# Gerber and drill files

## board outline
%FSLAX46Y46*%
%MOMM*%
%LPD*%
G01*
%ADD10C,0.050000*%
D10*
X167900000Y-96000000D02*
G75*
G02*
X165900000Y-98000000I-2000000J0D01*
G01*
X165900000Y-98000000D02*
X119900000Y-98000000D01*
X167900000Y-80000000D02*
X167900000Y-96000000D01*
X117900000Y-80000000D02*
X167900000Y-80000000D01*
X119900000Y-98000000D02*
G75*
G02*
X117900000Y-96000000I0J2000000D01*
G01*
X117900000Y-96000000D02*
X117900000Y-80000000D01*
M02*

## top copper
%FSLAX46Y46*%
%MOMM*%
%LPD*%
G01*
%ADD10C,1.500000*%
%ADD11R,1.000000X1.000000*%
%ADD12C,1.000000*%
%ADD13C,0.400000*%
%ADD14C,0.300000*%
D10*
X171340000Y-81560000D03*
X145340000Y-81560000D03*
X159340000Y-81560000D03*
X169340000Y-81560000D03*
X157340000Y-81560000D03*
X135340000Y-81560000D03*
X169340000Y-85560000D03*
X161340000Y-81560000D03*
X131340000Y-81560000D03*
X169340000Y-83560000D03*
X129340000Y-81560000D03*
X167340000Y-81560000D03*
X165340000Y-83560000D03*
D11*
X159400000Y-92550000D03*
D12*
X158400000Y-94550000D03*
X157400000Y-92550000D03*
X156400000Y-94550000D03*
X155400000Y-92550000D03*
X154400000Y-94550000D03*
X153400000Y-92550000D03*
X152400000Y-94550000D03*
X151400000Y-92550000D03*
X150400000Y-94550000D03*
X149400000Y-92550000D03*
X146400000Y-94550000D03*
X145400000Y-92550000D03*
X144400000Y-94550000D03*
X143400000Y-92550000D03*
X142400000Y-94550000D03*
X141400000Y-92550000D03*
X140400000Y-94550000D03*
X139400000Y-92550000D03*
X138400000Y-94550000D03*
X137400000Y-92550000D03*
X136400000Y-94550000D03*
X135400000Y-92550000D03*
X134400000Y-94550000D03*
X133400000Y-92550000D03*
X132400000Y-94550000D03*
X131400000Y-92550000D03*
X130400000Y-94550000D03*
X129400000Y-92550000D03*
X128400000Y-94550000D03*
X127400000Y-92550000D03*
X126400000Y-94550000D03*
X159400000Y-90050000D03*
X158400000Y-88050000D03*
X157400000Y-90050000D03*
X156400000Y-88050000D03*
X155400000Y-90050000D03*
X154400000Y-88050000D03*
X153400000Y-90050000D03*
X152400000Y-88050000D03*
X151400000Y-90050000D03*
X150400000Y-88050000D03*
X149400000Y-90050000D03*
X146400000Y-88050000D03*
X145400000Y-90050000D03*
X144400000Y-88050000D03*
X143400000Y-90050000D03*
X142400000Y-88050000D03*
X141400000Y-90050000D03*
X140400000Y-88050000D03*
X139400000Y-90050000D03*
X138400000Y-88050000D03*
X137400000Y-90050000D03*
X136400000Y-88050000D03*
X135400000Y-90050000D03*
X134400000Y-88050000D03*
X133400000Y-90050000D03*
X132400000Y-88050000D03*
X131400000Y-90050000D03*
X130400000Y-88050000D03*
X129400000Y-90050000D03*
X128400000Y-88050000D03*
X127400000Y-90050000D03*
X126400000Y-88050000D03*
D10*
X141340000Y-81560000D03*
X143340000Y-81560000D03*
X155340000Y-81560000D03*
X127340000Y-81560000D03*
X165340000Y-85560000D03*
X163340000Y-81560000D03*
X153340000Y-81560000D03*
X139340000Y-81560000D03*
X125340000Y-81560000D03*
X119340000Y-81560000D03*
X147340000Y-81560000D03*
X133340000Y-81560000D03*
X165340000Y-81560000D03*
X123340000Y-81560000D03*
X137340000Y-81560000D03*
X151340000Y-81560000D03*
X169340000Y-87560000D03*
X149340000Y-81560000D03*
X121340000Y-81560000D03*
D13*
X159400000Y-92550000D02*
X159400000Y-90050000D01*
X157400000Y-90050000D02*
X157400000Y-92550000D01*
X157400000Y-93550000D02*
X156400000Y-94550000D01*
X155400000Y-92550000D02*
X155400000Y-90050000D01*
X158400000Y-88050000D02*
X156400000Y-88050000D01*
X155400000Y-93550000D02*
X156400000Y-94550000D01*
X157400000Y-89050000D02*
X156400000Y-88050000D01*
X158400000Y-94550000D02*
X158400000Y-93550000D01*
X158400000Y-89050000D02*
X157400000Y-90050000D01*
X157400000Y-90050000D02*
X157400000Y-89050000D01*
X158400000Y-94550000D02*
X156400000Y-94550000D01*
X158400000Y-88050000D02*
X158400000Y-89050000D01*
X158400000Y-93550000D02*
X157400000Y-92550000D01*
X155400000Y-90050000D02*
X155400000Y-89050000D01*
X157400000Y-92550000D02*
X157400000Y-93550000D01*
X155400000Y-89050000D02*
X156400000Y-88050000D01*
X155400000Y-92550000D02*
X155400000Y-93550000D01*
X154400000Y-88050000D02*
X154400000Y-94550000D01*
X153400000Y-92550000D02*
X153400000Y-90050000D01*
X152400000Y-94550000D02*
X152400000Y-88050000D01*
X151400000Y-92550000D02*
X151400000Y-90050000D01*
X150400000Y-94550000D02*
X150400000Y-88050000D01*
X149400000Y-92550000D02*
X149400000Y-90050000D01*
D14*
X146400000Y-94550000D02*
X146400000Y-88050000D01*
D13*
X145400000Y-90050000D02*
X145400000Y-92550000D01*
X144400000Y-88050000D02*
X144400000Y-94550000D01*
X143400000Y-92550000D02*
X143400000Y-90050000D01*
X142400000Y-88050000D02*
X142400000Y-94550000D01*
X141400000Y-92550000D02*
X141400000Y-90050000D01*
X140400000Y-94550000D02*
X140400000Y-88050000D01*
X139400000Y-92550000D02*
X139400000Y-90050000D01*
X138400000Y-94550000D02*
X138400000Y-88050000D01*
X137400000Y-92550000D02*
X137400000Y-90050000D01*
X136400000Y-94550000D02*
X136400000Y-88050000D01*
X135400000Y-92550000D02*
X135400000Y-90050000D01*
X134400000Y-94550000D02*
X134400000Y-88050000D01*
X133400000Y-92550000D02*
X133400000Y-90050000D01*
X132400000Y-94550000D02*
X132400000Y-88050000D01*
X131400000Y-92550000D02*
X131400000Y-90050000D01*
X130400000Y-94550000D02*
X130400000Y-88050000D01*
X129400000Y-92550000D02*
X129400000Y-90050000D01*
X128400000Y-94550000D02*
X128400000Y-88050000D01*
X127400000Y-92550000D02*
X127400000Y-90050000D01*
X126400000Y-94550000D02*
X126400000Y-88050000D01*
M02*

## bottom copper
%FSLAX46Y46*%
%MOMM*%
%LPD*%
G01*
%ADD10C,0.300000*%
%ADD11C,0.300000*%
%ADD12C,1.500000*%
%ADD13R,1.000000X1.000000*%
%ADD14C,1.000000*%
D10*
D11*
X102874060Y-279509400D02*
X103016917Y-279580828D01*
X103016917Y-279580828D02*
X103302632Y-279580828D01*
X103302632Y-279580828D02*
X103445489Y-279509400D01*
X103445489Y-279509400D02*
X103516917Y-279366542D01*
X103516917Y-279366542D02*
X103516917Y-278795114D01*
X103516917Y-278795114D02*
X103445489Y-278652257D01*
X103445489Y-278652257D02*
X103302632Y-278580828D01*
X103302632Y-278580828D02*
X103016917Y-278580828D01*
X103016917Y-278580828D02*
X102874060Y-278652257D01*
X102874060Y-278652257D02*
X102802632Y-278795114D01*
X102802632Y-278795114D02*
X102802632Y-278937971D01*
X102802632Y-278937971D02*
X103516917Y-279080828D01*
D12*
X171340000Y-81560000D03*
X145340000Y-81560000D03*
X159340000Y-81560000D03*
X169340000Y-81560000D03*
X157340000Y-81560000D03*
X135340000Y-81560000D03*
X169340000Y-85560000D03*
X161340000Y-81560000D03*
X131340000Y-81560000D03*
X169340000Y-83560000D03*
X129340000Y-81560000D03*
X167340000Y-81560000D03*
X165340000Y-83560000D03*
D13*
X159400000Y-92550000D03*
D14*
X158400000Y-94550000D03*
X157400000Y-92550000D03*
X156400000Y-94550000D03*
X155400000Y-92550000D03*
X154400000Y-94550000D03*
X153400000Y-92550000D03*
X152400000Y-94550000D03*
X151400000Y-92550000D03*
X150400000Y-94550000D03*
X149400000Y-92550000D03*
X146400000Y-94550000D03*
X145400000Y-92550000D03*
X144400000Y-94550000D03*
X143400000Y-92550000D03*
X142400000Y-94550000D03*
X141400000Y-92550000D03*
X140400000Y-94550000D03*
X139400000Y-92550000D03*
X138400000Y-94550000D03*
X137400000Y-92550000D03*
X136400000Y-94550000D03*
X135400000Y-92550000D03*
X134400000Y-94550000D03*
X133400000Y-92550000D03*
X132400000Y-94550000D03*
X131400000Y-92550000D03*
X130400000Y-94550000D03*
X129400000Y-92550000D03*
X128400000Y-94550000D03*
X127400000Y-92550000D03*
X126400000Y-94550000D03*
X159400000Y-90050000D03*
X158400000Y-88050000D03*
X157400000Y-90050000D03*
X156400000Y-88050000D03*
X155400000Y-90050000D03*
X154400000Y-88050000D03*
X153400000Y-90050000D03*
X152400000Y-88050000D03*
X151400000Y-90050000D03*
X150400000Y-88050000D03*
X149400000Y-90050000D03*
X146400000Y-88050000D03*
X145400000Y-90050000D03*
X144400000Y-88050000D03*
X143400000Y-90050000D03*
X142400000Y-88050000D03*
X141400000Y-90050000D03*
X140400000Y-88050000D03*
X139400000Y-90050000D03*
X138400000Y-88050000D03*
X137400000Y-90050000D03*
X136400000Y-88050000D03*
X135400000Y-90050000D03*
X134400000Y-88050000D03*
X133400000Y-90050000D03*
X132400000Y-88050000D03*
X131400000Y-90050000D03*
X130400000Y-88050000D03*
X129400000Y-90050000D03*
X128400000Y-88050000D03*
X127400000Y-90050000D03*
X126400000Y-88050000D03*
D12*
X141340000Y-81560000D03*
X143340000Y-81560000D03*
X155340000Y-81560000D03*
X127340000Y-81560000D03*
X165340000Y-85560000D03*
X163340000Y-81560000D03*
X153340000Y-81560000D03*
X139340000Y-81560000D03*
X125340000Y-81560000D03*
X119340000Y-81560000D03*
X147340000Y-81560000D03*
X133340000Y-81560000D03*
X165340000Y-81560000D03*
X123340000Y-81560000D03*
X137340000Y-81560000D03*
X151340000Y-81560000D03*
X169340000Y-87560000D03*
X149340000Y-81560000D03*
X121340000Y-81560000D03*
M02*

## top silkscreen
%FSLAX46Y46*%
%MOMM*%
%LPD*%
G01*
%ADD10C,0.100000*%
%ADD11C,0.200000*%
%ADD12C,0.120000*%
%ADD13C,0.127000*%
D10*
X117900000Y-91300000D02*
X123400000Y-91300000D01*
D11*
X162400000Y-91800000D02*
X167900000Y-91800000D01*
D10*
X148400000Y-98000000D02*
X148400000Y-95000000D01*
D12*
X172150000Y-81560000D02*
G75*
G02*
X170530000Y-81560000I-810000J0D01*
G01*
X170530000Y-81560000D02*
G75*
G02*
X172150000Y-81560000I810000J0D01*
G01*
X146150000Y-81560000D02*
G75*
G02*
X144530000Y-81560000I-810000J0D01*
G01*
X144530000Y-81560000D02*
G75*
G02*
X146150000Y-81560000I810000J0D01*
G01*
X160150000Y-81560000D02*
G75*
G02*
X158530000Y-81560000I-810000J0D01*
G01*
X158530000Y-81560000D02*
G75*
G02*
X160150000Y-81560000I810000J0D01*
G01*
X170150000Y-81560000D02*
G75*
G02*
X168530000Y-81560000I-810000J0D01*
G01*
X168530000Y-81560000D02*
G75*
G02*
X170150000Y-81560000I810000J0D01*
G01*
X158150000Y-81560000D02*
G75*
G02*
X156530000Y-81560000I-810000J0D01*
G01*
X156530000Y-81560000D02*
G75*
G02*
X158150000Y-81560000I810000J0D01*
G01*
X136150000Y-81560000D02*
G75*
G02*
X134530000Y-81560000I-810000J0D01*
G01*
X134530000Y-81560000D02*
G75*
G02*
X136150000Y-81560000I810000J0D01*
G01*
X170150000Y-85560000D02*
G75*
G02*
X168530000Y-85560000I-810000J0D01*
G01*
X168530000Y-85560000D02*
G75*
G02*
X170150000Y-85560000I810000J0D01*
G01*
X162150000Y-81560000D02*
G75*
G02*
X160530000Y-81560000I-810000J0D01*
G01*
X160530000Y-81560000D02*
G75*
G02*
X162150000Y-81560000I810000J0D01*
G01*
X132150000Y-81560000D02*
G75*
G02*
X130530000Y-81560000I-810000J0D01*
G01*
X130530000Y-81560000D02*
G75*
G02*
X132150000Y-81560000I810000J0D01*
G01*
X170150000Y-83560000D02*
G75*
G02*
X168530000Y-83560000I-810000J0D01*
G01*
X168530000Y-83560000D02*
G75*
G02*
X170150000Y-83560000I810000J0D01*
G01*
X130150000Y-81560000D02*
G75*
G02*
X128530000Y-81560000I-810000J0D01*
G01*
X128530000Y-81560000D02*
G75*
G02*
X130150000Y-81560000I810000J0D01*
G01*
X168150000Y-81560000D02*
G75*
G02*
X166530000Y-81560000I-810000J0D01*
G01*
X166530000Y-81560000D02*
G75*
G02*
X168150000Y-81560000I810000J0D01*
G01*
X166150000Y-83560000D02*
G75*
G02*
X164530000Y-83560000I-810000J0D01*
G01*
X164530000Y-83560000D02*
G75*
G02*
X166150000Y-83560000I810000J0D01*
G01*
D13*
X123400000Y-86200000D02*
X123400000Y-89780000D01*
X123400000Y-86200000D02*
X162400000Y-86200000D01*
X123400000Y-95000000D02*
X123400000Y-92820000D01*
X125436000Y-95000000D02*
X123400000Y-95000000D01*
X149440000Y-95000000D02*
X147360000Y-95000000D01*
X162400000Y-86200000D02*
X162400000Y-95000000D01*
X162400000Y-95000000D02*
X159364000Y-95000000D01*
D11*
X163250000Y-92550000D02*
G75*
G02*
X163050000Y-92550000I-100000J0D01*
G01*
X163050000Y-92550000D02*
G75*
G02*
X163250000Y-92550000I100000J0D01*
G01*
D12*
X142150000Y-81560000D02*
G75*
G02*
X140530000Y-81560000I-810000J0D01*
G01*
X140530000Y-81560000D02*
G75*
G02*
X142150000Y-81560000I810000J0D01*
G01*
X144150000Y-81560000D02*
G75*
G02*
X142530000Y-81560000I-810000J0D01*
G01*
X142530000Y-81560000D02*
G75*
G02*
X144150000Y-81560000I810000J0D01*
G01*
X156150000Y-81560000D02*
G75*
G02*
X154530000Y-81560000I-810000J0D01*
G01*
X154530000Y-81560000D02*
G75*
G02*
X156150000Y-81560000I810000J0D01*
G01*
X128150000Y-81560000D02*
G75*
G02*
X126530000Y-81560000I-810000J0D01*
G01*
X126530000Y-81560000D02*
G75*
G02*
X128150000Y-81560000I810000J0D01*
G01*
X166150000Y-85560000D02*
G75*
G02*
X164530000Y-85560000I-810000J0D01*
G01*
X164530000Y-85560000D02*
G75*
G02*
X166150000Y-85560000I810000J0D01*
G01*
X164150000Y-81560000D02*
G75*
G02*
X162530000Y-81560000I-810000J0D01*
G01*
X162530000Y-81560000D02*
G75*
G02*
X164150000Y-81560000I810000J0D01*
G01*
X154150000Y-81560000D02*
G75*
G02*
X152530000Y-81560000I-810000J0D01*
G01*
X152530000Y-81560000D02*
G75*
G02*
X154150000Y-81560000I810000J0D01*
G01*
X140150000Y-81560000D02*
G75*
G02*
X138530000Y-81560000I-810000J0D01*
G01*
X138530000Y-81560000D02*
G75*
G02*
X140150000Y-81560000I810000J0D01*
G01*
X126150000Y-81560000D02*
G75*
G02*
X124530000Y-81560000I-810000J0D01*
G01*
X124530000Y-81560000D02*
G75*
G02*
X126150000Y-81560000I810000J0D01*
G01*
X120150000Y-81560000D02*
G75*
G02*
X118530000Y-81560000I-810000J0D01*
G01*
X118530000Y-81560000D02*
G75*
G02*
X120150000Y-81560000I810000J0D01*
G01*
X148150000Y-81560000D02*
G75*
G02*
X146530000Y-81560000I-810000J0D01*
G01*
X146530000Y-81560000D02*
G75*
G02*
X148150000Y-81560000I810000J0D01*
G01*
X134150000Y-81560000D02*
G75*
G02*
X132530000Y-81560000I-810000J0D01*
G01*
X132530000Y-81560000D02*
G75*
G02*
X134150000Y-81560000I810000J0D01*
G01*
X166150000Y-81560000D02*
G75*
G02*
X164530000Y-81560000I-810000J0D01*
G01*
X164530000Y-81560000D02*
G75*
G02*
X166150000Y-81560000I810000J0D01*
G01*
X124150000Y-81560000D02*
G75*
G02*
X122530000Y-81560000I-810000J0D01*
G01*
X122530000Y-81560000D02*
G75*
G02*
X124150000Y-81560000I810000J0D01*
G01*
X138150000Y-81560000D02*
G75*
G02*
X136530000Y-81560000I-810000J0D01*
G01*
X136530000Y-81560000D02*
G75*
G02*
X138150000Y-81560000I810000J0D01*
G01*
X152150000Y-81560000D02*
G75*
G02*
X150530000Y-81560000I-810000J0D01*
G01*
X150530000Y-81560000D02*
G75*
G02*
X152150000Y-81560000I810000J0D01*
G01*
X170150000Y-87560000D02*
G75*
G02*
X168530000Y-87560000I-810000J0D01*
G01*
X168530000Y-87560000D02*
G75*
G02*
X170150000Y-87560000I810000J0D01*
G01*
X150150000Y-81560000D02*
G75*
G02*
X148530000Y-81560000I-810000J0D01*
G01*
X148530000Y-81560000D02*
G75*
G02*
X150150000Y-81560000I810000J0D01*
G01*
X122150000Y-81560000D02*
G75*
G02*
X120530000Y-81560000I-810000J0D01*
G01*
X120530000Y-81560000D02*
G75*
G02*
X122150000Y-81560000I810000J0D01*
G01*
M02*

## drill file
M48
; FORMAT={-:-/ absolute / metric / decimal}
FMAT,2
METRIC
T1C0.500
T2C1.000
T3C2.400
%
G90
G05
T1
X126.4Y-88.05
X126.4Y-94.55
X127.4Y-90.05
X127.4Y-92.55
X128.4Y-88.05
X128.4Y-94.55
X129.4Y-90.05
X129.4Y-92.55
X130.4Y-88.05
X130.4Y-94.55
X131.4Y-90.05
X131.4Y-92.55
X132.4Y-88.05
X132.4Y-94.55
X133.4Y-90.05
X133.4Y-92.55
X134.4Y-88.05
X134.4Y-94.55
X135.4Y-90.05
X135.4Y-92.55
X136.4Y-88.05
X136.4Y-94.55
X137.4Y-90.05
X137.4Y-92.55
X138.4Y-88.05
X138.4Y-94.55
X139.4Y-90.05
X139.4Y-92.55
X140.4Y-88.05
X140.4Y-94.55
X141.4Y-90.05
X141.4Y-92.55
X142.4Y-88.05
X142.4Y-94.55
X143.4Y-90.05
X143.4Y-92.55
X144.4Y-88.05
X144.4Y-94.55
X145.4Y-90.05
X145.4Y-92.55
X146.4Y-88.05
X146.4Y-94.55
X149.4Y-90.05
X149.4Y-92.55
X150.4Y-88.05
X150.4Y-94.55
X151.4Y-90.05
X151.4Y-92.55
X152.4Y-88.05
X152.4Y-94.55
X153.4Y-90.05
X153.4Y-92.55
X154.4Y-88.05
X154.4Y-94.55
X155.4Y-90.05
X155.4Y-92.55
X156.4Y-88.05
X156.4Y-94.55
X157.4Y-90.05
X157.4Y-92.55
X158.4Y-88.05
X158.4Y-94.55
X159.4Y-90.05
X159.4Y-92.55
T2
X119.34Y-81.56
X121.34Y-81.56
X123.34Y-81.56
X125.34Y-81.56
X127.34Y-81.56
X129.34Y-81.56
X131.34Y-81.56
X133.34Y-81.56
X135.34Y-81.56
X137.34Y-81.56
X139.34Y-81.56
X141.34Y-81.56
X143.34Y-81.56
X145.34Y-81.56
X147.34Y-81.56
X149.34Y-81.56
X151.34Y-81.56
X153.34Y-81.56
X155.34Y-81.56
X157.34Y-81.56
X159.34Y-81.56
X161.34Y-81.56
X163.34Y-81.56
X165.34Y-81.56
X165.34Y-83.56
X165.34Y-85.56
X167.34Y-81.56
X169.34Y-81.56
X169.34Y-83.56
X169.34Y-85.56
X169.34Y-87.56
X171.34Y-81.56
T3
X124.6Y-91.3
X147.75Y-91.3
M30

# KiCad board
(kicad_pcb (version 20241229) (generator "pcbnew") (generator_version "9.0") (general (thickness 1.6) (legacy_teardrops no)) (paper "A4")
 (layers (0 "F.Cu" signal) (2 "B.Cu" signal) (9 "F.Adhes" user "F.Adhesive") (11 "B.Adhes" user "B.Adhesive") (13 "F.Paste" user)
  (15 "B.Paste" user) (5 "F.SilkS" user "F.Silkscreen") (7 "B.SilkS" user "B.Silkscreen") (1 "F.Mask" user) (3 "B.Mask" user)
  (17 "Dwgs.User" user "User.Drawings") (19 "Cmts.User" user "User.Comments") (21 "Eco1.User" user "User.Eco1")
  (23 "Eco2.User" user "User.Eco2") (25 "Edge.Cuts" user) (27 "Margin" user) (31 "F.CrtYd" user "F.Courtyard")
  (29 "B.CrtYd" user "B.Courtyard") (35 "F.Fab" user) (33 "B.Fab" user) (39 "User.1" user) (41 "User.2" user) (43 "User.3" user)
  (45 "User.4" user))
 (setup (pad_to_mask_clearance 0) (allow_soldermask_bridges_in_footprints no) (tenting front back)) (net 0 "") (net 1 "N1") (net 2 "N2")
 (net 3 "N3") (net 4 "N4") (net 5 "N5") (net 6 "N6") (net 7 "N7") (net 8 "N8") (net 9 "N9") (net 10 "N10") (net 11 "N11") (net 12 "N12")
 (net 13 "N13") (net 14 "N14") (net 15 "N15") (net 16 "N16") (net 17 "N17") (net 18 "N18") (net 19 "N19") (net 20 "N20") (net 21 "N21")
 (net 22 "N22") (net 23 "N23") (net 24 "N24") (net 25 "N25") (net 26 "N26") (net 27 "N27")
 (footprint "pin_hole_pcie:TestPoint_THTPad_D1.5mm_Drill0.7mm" (layer "F.Cu") (at 171.34 81.56 90)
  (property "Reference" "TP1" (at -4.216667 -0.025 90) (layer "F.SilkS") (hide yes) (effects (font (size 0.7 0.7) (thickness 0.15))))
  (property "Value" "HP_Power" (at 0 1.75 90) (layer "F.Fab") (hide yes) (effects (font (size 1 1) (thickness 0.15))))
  (fp_circle (center 0 0) (end 0 0.81) (stroke (width 0.12) (type solid)) (fill no) (layer "F.SilkS"))
  (pad "1" thru_hole circle (at 0 0 90) (size 1.5 1.5) (drill 1) (layers "*.Cu" "*.Mask") (remove_unused_layers no) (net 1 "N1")))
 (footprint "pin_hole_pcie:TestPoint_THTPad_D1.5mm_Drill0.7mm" (layer "F.Cu") (at 145.34 81.56 90)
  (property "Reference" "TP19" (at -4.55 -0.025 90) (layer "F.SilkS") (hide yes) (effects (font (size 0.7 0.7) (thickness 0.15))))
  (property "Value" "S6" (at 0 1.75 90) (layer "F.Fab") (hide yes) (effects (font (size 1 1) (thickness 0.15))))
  (fp_circle (center 0 0) (end 0 0.81) (stroke (width 0.12) (type solid)) (fill no) (layer "F.SilkS"))
  (pad "1" thru_hole circle (at 0 0 90) (size 1.5 1.5) (drill 1) (layers "*.Cu" "*.Mask") (remove_unused_layers no) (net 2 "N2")))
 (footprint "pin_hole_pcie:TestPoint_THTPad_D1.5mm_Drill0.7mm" (layer "F.Cu") (at 159.34 81.56 90)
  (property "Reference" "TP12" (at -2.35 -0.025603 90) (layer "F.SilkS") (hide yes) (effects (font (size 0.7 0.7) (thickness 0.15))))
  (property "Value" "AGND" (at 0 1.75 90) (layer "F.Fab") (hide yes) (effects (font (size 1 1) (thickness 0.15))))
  (fp_circle (center 0 0) (end 0 0.81) (stroke (width 0.12) (type solid)) (fill no) (layer "F.SilkS"))
  (pad "1" thru_hole circle (at 0 0 90) (size 1.5 1.5) (drill 1) (layers "*.Cu" "*.Mask") (remove_unused_layers no) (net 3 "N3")))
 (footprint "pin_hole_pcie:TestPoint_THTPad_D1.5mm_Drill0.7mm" (layer "F.Cu") (at 169.34 81.56 90)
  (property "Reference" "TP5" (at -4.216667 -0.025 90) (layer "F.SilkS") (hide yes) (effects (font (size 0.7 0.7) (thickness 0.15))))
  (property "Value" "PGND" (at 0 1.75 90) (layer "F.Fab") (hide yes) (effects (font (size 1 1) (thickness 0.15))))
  (fp_circle (center 0 0) (end 0 0.81) (stroke (width 0.12) (type solid)) (fill no) (layer "F.SilkS"))
  (pad "1" thru_hole circle (at 0 0 90) (size 1.5 1.5) (drill 1) (layers "*.Cu" "*.Mask") (remove_unused_layers no) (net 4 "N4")))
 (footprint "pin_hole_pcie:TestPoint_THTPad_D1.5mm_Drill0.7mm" (layer "F.Cu") (at 157.34 81.56 90)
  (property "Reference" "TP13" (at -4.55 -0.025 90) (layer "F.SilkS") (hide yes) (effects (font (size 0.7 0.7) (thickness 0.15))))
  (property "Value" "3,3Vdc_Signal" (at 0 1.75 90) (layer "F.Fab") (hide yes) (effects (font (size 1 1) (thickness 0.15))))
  (fp_circle (center 0 0) (end 0 0.81) (stroke (width 0.12) (type solid)) (fill no) (layer "F.SilkS"))
  (pad "1" thru_hole circle (at 0 0 90) (size 1.5 1.5) (drill 1) (layers "*.Cu" "*.Mask") (remove_unused_layers no) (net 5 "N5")))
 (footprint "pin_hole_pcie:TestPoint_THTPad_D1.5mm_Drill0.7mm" (layer "F.Cu") (at 135.34 81.56 90)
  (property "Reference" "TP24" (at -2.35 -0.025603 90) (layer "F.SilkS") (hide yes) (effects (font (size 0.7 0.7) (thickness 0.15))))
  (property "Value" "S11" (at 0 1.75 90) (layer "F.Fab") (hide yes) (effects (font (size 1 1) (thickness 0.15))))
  (fp_circle (center 0 0) (end 0 0.81) (stroke (width 0.12) (type solid)) (fill no) (layer "F.SilkS"))
  (pad "1" thru_hole circle (at 0 0 90) (size 1.5 1.5) (drill 1) (layers "*.Cu" "*.Mask") (remove_unused_layers no) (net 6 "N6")))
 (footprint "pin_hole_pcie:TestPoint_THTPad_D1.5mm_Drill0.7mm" (layer "F.Cu") (at 169.34 85.56 90)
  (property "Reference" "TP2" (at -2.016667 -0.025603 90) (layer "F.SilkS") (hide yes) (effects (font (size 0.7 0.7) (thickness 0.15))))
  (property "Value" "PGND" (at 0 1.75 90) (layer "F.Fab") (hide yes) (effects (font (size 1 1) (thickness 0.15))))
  (fp_circle (center 0 0) (end 0 0.81) (stroke (width 0.12) (type solid)) (fill no) (layer "F.SilkS"))
  (pad "1" thru_hole circle (at 0 0 90) (size 1.5 1.5) (drill 1) (layers "*.Cu" "*.Mask") (remove_unused_layers no) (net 4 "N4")))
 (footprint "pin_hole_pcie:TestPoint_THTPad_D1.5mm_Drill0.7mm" (layer "F.Cu") (at 161.34 81.56 90)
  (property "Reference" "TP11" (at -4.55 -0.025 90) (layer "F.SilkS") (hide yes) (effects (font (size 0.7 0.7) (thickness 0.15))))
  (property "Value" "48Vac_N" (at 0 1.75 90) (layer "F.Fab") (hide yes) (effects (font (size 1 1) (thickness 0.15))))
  (fp_circle (center 0 0) (end 0 0.81) (stroke (width 0.12) (type solid)) (fill no) (layer "F.SilkS"))
  (pad "1" thru_hole circle (at 0 0 90) (size 1.5 1.5) (drill 1) (layers "*.Cu" "*.Mask") (remove_unused_layers no) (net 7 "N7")))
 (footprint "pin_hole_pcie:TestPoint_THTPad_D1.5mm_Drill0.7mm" (layer "F.Cu") (at 131.34 81.56 90)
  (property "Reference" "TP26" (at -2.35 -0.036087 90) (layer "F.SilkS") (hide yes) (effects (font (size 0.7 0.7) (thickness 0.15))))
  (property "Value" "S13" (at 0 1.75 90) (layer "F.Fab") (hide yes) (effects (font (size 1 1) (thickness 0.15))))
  (fp_circle (center 0 0) (end 0 0.81) (stroke (width 0.12) (type solid)) (fill no) (layer "F.SilkS"))
  (pad "1" thru_hole circle (at 0 0 90) (size 1.5 1.5) (drill 1) (layers "*.Cu" "*.Mask") (remove_unused_layers no) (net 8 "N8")))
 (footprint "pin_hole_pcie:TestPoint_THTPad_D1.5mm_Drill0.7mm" (layer "F.Cu") (at 169.34 83.56 90)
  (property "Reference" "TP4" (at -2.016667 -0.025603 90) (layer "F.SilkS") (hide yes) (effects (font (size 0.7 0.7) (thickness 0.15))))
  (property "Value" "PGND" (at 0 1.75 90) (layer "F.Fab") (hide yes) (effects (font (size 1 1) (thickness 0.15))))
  (fp_circle (center 0 0) (end 0 0.81) (stroke (width 0.12) (type solid)) (fill no) (layer "F.SilkS"))
  (pad "1" thru_hole circle (at 0 0 90) (size 1.5 1.5) (drill 1) (layers "*.Cu" "*.Mask") (remove_unused_layers no) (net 4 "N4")))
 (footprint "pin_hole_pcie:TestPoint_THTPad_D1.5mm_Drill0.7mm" (layer "F.Cu") (at 129.34 81.56 90)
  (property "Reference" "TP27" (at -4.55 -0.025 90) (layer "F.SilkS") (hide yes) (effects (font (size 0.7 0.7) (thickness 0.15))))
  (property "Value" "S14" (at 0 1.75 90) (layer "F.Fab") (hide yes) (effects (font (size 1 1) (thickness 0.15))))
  (fp_circle (center 0 0) (end 0 0.81) (stroke (width 0.12) (type solid)) (fill no) (layer "F.SilkS"))
  (pad "1" thru_hole circle (at 0 0 90) (size 1.5 1.5) (drill 1) (layers "*.Cu" "*.Mask") (remove_unused_layers no) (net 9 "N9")))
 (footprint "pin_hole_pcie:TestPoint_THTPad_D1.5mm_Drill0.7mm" (layer "F.Cu") (at 167.34 81.56 90)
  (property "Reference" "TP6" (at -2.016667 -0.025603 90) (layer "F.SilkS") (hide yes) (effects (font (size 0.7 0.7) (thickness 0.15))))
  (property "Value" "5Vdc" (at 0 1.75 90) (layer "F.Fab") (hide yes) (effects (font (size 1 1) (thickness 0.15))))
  (fp_circle (center 0 0) (end 0 0.81) (stroke (width 0.12) (type solid)) (fill no) (layer "F.SilkS"))
  (pad "1" thru_hole circle (at 0 0 90) (size 1.5 1.5) (drill 1) (layers "*.Cu" "*.Mask") (remove_unused_layers no) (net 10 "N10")))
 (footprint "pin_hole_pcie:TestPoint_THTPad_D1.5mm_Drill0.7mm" (layer "F.Cu") (at 165.34 83.56 90)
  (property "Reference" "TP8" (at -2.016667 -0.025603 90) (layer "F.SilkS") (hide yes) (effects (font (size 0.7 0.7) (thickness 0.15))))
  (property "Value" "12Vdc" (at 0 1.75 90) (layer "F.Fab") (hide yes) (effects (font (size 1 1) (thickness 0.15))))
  (fp_circle (center 0 0) (end 0 0.81) (stroke (width 0.12) (type solid)) (fill no) (layer "F.SilkS"))
  (pad "1" thru_hole circle (at 0 0 90) (size 1.5 1.5) (drill 1) (layers "*.Cu" "*.Mask") (remove_unused_layers no) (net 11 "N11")))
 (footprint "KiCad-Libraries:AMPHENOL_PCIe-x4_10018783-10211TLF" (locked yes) (layer "F.Cu") (at 147.75 91.3 180)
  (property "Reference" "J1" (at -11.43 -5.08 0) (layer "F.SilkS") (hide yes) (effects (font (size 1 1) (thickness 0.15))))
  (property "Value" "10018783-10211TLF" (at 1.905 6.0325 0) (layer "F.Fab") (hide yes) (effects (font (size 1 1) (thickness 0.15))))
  (fp_line (start 24.35 5.1) (end 24.35 1.52) (stroke (width 0.127) (type solid)) (layer "F.SilkS"))
  (fp_line (start 24.35 5.1) (end -14.65 5.1) (stroke (width 0.127) (type solid)) (layer "F.SilkS"))
  (fp_line (start 24.35 -3.7) (end 24.35 -1.52) (stroke (width 0.127) (type solid)) (layer "F.SilkS"))
  (fp_line (start 22.314 -3.7) (end 24.35 -3.7) (stroke (width 0.127) (type solid)) (layer "F.SilkS"))
  (fp_line (start -1.69 -3.7) (end 0.39 -3.7) (stroke (width 0.127) (type solid)) (layer "F.SilkS"))
  (fp_line (start -14.65 5.1) (end -14.65 -3.7) (stroke (width 0.127) (type solid)) (layer "F.SilkS"))
  (fp_line (start -14.65 -3.7) (end -11.614 -3.7) (stroke (width 0.127) (type solid)) (layer "F.SilkS"))
  (fp_circle (center -15.4 -1.25) (end -15.3 -1.25) (stroke (width 0.2) (type solid)) (fill no) (layer "F.SilkS"))
  (pad "" np_thru_hole circle (at 0 0 180) (size 1 2.4) (drill 2.4) (layers "*.Cu" "*.Mask"))
  (pad "" np_thru_hole circle (at 23.15 0 180) (size 1 2.4) (drill 2.4) (layers "*.Cu" "*.Mask"))
  (pad "A1" thru_hole rect (at -11.65 -1.25 180) (size 1 1) (drill 0.5) (layers "*.Cu" "*.Mask") (remove_unused_layers no) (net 1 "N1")
   (solder_mask_margin 0.102))
  (pad "A2" thru_hole circle (at -10.65 -3.25 180) (size 1 0.8) (drill 0.5) (layers "*.Cu" "*.Mask") (remove_unused_layers no) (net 4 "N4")
   (solder_mask_margin 0.102))
  (pad "A3" thru_hole circle (at -9.65 -1.25 180) (size 1 0.8) (drill 0.5) (layers "*.Cu" "*.Mask") (remove_unused_layers no) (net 4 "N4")
   (solder_mask_margin 0.102))
  (pad "A4" thru_hole circle (at -8.65 -3.25 180) (size 1 0.8) (drill 0.5) (layers "*.Cu" "*.Mask") (remove_unused_layers no) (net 4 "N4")
   (solder_mask_margin 0.102))
  (pad "A5" thru_hole circle (at -7.65 -1.25 180) (size 1 0.8) (drill 0.5) (layers "*.Cu" "*.Mask") (remove_unused_layers no) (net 4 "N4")
   (solder_mask_margin 0.102))
  (pad "A6" thru_hole circle (at -6.65 -3.25 180) (size 1 0.8) (drill 0.5) (layers "*.Cu" "*.Mask") (remove_unused_layers no) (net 10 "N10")
   (solder_mask_margin 0.102))
  (pad "A7" thru_hole circle (at -5.65 -1.25 180) (size 1 0.8) (drill 0.5) (layers "*.Cu" "*.Mask") (remove_unused_layers no) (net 11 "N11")
   (solder_mask_margin 0.102))
  (pad "A8" thru_hole circle (at -4.65 -3.25 180) (size 1 0.8) (drill 0.5) (layers "*.Cu" "*.Mask") (remove_unused_layers no) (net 11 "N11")
   (solder_mask_margin 0.102))
  (pad "A9" thru_hole circle (at -3.65 -1.25 180) (size 1 0.8) (drill 0.5) (layers "*.Cu" "*.Mask") (remove_unused_layers no) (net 11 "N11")
   (solder_mask_margin 0.102))
  (pad "A10" thru_hole circle (at -2.65 -3.25 180) (size 1 0.8) (drill 0.5) (layers "*.Cu" "*.Mask") (remove_unused_layers no)
   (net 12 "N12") (solder_mask_margin 0.102))
  (pad "A11" thru_hole circle (at -1.65 -1.25 180) (size 1 0.8) (drill 0.5) (layers "*.Cu" "*.Mask") (remove_unused_layers no) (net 7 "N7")
   (solder_mask_margin 0.102))
  (pad "A12" thru_hole circle (at 1.35 -3.25 180) (size 1 0.8) (drill 0.5) (layers "*.Cu" "*.Mask") (remove_unused_layers no) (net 3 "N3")
   (solder_mask_margin 0.102))
  (pad "A13" thru_hole circle (at 2.35 -1.25 180) (size 1 0.8) (drill 0.5) (layers "*.Cu" "*.Mask") (remove_unused_layers no) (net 5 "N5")
   (solder_mask_margin 0.102))
  (pad "A14" thru_hole circle (at 3.35 -3.25 180) (size 1 0.8) (drill 0.5) (layers "*.Cu" "*.Mask") (remove_unused_layers no) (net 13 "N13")
   (solder_mask_margin 0.102))
  (pad "A15" thru_hole circle (at 4.35 -1.25 180) (size 1 0.8) (drill 0.5) (layers "*.Cu" "*.Mask") (remove_unused_layers no) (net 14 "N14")
   (solder_mask_margin 0.102))
  (pad "A16" thru_hole circle (at 5.35 -3.25 180) (size 1 0.8) (drill 0.5) (layers "*.Cu" "*.Mask") (remove_unused_layers no) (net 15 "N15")
   (solder_mask_margin 0.102))
  (pad "A17" thru_hole circle (at 6.35 -1.25 180) (size 1 0.8) (drill 0.5) (layers "*.Cu" "*.Mask") (remove_unused_layers no) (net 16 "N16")
   (solder_mask_margin 0.102))
  (pad "A18" thru_hole circle (at 7.35 -3.25 180) (size 1 0.8) (drill 0.5) (layers "*.Cu" "*.Mask") (remove_unused_layers no) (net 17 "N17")
   (solder_mask_margin 0.102))
  (pad "A19" thru_hole circle (at 8.35 -1.25 180) (size 1 0.8) (drill 0.5) (layers "*.Cu" "*.Mask") (remove_unused_layers no) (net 2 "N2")
   (solder_mask_margin 0.102))
  (pad "A20" thru_hole circle (at 9.35 -3.25 180) (size 1 0.8) (drill 0.5) (layers "*.Cu" "*.Mask") (remove_unused_layers no) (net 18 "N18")
   (solder_mask_margin 0.102))
  (pad "A21" thru_hole circle (at 10.35 -1.25 180) (size 1 0.8) (drill 0.5) (layers "*.Cu" "*.Mask") (remove_unused_layers no)
   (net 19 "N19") (solder_mask_margin 0.102))
  (pad "A22" thru_hole circle (at 11.35 -3.25 180) (size 1 0.8) (drill 0.5) (layers "*.Cu" "*.Mask") (remove_unused_layers no)
   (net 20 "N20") (solder_mask_margin 0.102))
  (pad "A23" thru_hole circle (at 12.35 -1.25 180) (size 1 0.8) (drill 0.5) (layers "*.Cu" "*.Mask") (remove_unused_layers no)
   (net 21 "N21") (solder_mask_margin 0.102))
  (pad "A24" thru_hole circle (at 13.35 -3.25 180) (size 1 0.8) (drill 0.5) (layers "*.Cu" "*.Mask") (remove_unused_layers no) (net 6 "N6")
   (solder_mask_margin 0.102))
  (pad "A25" thru_hole circle (at 14.35 -1.25 180) (size 1 0.8) (drill 0.5) (layers "*.Cu" "*.Mask") (remove_unused_layers no)
   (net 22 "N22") (solder_mask_margin 0.102))
  (pad "A26" thru_hole circle (at 15.35 -3.25 180) (size 1 0.8) (drill 0.5) (layers "*.Cu" "*.Mask") (remove_unused_layers no) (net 8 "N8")
   (solder_mask_margin 0.102))
  (pad "A27" thru_hole circle (at 16.35 -1.25 180) (size 1 0.8) (drill 0.5) (layers "*.Cu" "*.Mask") (remove_unused_layers no) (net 9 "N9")
   (solder_mask_margin 0.102))
  (pad "A28" thru_hole circle (at 17.35 -3.25 180) (size 1 0.8) (drill 0.5) (layers "*.Cu" "*.Mask") (remove_unused_layers no)
   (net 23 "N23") (solder_mask_margin 0.102))
  (pad "A29" thru_hole circle (at 18.35 -1.25 180) (size 1 0.8) (drill 0.5) (layers "*.Cu" "*.Mask") (remove_unused_layers no)
   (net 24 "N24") (solder_mask_margin 0.102))
  (pad "A30" thru_hole circle (at 19.35 -3.25 180) (size 1 0.8) (drill 0.5) (layers "*.Cu" "*.Mask") (remove_unused_layers no)
   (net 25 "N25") (solder_mask_margin 0.102))
  (pad "A31" thru_hole circle (at 20.35 -1.25 180) (size 1 0.8) (drill 0.5) (layers "*.Cu" "*.Mask") (remove_unused_layers no)
   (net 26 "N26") (solder_mask_margin 0.102))
  (pad "A32" thru_hole circle (at 21.35 -3.25 180) (size 1 1) (drill 0.5) (layers "*.Cu" "*.Mask") (remove_unused_layers no) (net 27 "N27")
   (solder_mask_margin 0.102))
  (pad "B1" thru_hole circle (at -11.65 1.25 180) (size 1 0.8) (drill 0.5) (layers "*.Cu" "*.Mask") (remove_unused_layers no) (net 1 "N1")
   (solder_mask_margin 0.102))
  (pad "B2" thru_hole circle (at -10.65 3.25 180) (size 1 0.8) (drill 0.5) (layers "*.Cu" "*.Mask") (remove_unused_layers no) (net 4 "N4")
   (solder_mask_margin 0.102))
  (pad "B3" thru_hole circle (at -9.65 1.25 180) (size 1 0.8) (drill 0.5) (layers "*.Cu" "*.Mask") (remove_unused_layers no) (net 4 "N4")
   (solder_mask_margin 0.102))
  (pad "B4" thru_hole circle (at -8.65 3.25 180) (size 1 0.8) (drill 0.5) (layers "*.Cu" "*.Mask") (remove_unused_layers no) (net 4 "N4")
   (solder_mask_margin 0.102))
  (pad "B5" thru_hole circle (at -7.65 1.25 180) (size 1 0.8) (drill 0.5) (layers "*.Cu" "*.Mask") (remove_unused_layers no) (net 4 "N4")
   (solder_mask_margin 0.102))
  (pad "B6" thru_hole circle (at -6.65 3.25 180) (size 1 0.8) (drill 0.5) (layers "*.Cu" "*.Mask") (remove_unused_layers no) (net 10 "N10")
   (solder_mask_margin 0.102))
  (pad "B7" thru_hole circle (at -5.65 1.25 180) (size 1 0.8) (drill 0.5) (layers "*.Cu" "*.Mask") (remove_unused_layers no) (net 11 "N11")
   (solder_mask_margin 0.102))
  (pad "B8" thru_hole circle (at -4.65 3.25 180) (size 1 0.8) (drill 0.5) (layers "*.Cu" "*.Mask") (remove_unused_layers no) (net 11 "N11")
   (solder_mask_margin 0.102))
  (pad "B9" thru_hole circle (at -3.65 1.25 180) (size 1 0.8) (drill 0.5) (layers "*.Cu" "*.Mask") (remove_unused_layers no) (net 11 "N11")
   (solder_mask_margin 0.102))
  (pad "B10" thru_hole circle (at -2.65 3.25 180) (size 1 0.8) (drill 0.5) (layers "*.Cu" "*.Mask") (remove_unused_layers no) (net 12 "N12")
   (solder_mask_margin 0.102))
  (pad "B11" thru_hole circle (at -1.65 1.25 180) (size 1 0.8) (drill 0.5) (layers "*.Cu" "*.Mask") (remove_unused_layers no) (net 7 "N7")
   (solder_mask_margin 0.102))
  (pad "B12" thru_hole circle (at 1.35 3.25 180) (size 1 0.8) (drill 0.5) (layers "*.Cu" "*.Mask") (remove_unused_layers no) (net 3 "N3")
   (solder_mask_margin 0.102))
  (pad "B13" thru_hole circle (at 2.35 1.25 180) (size 1 0.8) (drill 0.5) (layers "*.Cu" "*.Mask") (remove_unused_layers no) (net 5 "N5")
   (solder_mask_margin 0.102))
  (pad "B14" thru_hole circle (at 3.35 3.25 180) (size 1 0.8) (drill 0.5) (layers "*.Cu" "*.Mask") (remove_unused_layers no) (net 13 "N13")
   (solder_mask_margin 0.102))
  (pad "B15" thru_hole circle (at 4.35 1.25 180) (size 1 0.8) (drill 0.5) (layers "*.Cu" "*.Mask") (remove_unused_layers no) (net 14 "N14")
   (solder_mask_margin 0.102))
  (pad "B16" thru_hole circle (at 5.35 3.25 180) (size 1 0.8) (drill 0.5) (layers "*.Cu" "*.Mask") (remove_unused_layers no) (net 15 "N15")
   (solder_mask_margin 0.102))
  (pad "B17" thru_hole circle (at 6.35 1.25 180) (size 1 0.8) (drill 0.5) (layers "*.Cu" "*.Mask") (remove_unused_layers no) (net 16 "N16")
   (solder_mask_margin 0.102))
  (pad "B18" thru_hole circle (at 7.35 3.25 180) (size 1 0.8) (drill 0.5) (layers "*.Cu" "*.Mask") (remove_unused_layers no) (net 17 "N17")
   (solder_mask_margin 0.102))
  (pad "B19" thru_hole circle (at 8.35 1.25 180) (size 1 0.8) (drill 0.5) (layers "*.Cu" "*.Mask") (remove_unused_layers no) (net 2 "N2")
   (solder_mask_margin 0.102))
  (pad "B20" thru_hole circle (at 9.35 3.25 180) (size 1 0.8) (drill 0.5) (layers "*.Cu" "*.Mask") (remove_unused_layers no) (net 18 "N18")
   (solder_mask_margin 0.102))
  (pad "B21" thru_hole circle (at 10.35 1.25 180) (size 1 0.8) (drill 0.5) (layers "*.Cu" "*.Mask") (remove_unused_layers no) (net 19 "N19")
   (solder_mask_margin 0.102))
  (pad "B22" thru_hole circle (at 11.35 3.25 180) (size 1 0.8) (drill 0.5) (layers "*.Cu" "*.Mask") (remove_unused_layers no) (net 20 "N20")
   (solder_mask_margin 0.102))
  (pad "B23" thru_hole circle (at 12.35 1.25 180) (size 1 0.8) (drill 0.5) (layers "*.Cu" "*.Mask") (remove_unused_layers no) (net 21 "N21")
   (solder_mask_margin 0.102))
  (pad "B24" thru_hole circle (at 13.35 3.25 180) (size 1 0.8) (drill 0.5) (layers "*.Cu" "*.Mask") (remove_unused_layers no) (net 6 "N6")
   (solder_mask_margin 0.102))
  (pad "B25" thru_hole circle (at 14.35 1.25 180) (size 1 0.8) (drill 0.5) (layers "*.Cu" "*.Mask") (remove_unused_layers no) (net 22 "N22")
   (solder_mask_margin 0.102))
  (pad "B26" thru_hole circle (at 15.35 3.25 180) (size 1 0.8) (drill 0.5) (layers "*.Cu" "*.Mask") (remove_unused_layers no) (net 8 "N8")
   (solder_mask_margin 0.102))
  (pad "B27" thru_hole circle (at 16.35 1.25 180) (size 1 0.8) (drill 0.5) (layers "*.Cu" "*.Mask") (remove_unused_layers no) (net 9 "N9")
   (solder_mask_margin 0.102))
  (pad "B28" thru_hole circle (at 17.35 3.25 180) (size 1 0.8) (drill 0.5) (layers "*.Cu" "*.Mask") (remove_unused_layers no) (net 23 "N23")
   (solder_mask_margin 0.102))
  (pad "B29" thru_hole circle (at 18.35 1.25 180) (size 1 0.8) (drill 0.5) (layers "*.Cu" "*.Mask") (remove_unused_layers no) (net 24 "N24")
   (solder_mask_margin 0.102))
  (pad "B30" thru_hole circle (at 19.35 3.25 180) (size 1 0.8) (drill 0.5) (layers "*.Cu" "*.Mask") (remove_unused_layers no) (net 25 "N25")
   (solder_mask_margin 0.102))
  (pad "B31" thru_hole circle (at 20.35 1.25 180) (size 1 0.8) (drill 0.5) (layers "*.Cu" "*.Mask") (remove_unused_layers no) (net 26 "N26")
   (solder_mask_margin 0.102))
  (pad "B32" thru_hole circle (at 21.35 3.25 180) (size 1 0.8) (drill 0.5) (layers "*.Cu" "*.Mask") (remove_unused_layers no) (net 27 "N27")
   (solder_mask_margin 0.102)))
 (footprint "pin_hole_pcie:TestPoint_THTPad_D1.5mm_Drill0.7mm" (layer "F.Cu") (at 141.34 81.56 90)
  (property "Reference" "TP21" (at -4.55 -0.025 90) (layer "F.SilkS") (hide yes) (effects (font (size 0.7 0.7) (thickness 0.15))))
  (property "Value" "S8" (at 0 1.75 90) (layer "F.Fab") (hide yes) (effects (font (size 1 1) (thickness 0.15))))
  (fp_circle (center 0 0) (end 0 0.81) (stroke (width 0.12) (type solid)) (fill no) (layer "F.SilkS"))
  (pad "1" thru_hole circle (at 0 0 90) (size 1.5 1.5) (drill 1) (layers "*.Cu" "*.Mask") (remove_unused_layers no) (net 19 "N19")))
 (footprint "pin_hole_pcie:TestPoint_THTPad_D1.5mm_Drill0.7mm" (layer "F.Cu") (at 143.34 81.56 90)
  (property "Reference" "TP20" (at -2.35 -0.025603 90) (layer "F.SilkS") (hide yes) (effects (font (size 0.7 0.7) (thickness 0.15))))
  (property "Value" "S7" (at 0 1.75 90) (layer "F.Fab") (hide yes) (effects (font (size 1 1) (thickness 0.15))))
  (fp_circle (center 0 0) (end 0 0.81) (stroke (width 0.12) (type solid)) (fill no) (layer "F.SilkS"))
  (pad "1" thru_hole circle (at 0 0 90) (size 1.5 1.5) (drill 1) (layers "*.Cu" "*.Mask") (remove_unused_layers no) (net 18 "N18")))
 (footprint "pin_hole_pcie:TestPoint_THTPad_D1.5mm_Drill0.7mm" (layer "F.Cu") (at 155.34 81.56 90)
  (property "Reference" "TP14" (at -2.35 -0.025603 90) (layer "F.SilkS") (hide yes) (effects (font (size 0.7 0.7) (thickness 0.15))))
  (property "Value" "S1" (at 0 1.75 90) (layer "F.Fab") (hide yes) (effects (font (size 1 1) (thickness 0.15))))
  (fp_circle (center 0 0) (end 0 0.81) (stroke (width 0.12) (type solid)) (fill no) (layer "F.SilkS"))
  (pad "1" thru_hole circle (at 0 0 90) (size 1.5 1.5) (drill 1) (layers "*.Cu" "*.Mask") (remove_unused_layers no) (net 13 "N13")))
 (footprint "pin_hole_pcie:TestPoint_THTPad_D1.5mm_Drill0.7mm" (layer "F.Cu") (at 127.34 81.56 90)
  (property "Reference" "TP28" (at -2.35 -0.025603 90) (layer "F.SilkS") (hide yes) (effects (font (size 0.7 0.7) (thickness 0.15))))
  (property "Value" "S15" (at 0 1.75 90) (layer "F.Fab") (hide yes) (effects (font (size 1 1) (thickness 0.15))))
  (fp_circle (center 0 0) (end 0 0.81) (stroke (width 0.12) (type solid)) (fill no) (layer "F.SilkS"))
  (pad "1" thru_hole circle (at 0 0 90) (size 1.5 1.5) (drill 1) (layers "*.Cu" "*.Mask") (remove_unused_layers no) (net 23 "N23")))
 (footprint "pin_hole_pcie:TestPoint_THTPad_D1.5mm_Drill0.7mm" (layer "F.Cu") (at 165.34 85.56 90)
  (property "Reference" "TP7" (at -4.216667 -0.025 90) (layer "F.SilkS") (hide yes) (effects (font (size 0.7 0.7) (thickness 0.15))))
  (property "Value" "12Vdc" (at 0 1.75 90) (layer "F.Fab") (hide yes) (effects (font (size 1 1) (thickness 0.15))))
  (fp_circle (center 0 0) (end 0 0.81) (stroke (width 0.12) (type solid)) (fill no) (layer "F.SilkS"))
  (pad "1" thru_hole circle (at 0 0 90) (size 1.5 1.5) (drill 1) (layers "*.Cu" "*.Mask") (remove_unused_layers no) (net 11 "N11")))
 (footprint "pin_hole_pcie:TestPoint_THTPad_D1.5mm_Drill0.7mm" (layer "F.Cu") (at 163.34 81.56 90)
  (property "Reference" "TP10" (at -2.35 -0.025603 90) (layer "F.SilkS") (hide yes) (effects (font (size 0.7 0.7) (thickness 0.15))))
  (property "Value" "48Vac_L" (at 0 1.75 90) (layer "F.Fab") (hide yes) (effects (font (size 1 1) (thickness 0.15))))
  (fp_circle (center 0 0) (end 0 0.81) (stroke (width 0.12) (type solid)) (fill no) (layer "F.SilkS"))
  (pad "1" thru_hole circle (at 0 0 90) (size 1.5 1.5) (drill 1) (layers "*.Cu" "*.Mask") (remove_unused_layers no) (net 12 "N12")))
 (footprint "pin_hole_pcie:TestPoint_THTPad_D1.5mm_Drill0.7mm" (layer "F.Cu") (at 153.34 81.56 90)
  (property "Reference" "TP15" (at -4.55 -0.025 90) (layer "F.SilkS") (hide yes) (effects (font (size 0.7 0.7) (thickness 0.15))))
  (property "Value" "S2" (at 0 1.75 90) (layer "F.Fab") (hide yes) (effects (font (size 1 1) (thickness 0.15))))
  (fp_circle (center 0 0) (end 0 0.81) (stroke (width 0.12) (type solid)) (fill no) (layer "F.SilkS"))
  (pad "1" thru_hole circle (at 0 0 90) (size 1.5 1.5) (drill 1) (layers "*.Cu" "*.Mask") (remove_unused_layers no) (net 14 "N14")))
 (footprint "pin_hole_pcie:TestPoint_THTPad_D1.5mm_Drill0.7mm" (layer "F.Cu") (at 139.34 81.56 90)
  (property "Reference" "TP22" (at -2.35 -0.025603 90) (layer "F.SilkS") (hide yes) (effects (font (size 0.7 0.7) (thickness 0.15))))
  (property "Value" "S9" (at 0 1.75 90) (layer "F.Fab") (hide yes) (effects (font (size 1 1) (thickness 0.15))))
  (fp_circle (center 0 0) (end 0 0.81) (stroke (width 0.12) (type solid)) (fill no) (layer "F.SilkS"))
  (pad "1" thru_hole circle (at 0 0 90) (size 1.5 1.5) (drill 1) (layers "*.Cu" "*.Mask") (remove_unused_layers no) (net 20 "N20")))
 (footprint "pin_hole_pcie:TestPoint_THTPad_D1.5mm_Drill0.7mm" (layer "F.Cu") (at 125.34 81.56 90)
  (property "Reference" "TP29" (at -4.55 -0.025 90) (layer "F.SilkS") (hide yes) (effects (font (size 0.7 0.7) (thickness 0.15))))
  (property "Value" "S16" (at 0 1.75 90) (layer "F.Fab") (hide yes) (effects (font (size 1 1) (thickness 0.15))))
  (fp_circle (center 0 0) (end 0 0.81) (stroke (width 0.12) (type solid)) (fill no) (layer "F.SilkS"))
  (pad "1" thru_hole circle (at 0 0 90) (size 1.5 1.5) (drill 1) (layers "*.Cu" "*.Mask") (remove_unused_layers no) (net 24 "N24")))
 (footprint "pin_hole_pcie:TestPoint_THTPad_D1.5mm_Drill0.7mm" (layer "F.Cu") (at 119.34 81.56 90)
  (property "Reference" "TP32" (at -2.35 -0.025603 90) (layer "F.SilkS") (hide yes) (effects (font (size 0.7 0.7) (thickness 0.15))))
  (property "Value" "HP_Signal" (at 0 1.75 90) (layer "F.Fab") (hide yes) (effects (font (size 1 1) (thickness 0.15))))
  (fp_circle (center 0 0) (end 0 0.81) (stroke (width 0.12) (type solid)) (fill no) (layer "F.SilkS"))
  (pad "1" thru_hole circle (at 0 0 90) (size 1.5 1.5) (drill 1) (layers "*.Cu" "*.Mask") (remove_unused_layers no) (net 27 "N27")))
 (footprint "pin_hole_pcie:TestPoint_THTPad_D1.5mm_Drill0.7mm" (layer "F.Cu") (at 147.34 81.56 90)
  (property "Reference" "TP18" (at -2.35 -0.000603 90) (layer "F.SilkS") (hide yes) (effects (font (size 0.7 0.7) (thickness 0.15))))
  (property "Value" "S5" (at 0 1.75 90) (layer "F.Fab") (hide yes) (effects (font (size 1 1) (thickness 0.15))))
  (fp_circle (center 0 0) (end 0 0.81) (stroke (width 0.12) (type solid)) (fill no) (layer "F.SilkS"))
  (pad "1" thru_hole circle (at 0 0 90) (size 1.5 1.5) (drill 1) (layers "*.Cu" "*.Mask") (remove_unused_layers no) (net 17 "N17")))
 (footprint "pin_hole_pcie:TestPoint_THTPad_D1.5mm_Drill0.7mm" (layer "F.Cu") (at 133.34 81.56 90)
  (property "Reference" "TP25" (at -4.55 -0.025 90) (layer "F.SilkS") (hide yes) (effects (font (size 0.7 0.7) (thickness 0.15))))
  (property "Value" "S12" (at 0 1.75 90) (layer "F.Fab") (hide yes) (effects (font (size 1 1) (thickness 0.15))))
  (fp_circle (center 0 0) (end 0 0.81) (stroke (width 0.12) (type solid)) (fill no) (layer "F.SilkS"))
  (pad "1" thru_hole circle (at 0 0 90) (size 1.5 1.5) (drill 1) (layers "*.Cu" "*.Mask") (remove_unused_layers no) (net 22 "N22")))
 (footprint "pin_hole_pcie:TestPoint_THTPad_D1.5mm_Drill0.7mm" (layer "F.Cu") (at 165.34 81.56 90)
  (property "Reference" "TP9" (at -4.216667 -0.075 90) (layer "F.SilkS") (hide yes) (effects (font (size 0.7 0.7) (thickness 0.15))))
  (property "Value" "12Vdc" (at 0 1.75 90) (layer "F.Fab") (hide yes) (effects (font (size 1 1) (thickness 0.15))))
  (fp_circle (center 0 0) (end 0 0.81) (stroke (width 0.12) (type solid)) (fill no) (layer "F.SilkS"))
  (pad "1" thru_hole circle (at 0 0 90) (size 1.5 1.5) (drill 1) (layers "*.Cu" "*.Mask") (remove_unused_layers no) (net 11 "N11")))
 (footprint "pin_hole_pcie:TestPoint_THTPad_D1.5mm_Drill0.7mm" (layer "F.Cu") (at 123.34 81.56 90)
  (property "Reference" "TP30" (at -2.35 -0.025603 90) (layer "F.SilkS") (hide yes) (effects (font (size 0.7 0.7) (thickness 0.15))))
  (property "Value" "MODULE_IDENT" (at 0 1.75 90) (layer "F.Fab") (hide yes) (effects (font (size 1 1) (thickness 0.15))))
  (fp_circle (center 0 0) (end 0 0.81) (stroke (width 0.12) (type solid)) (fill no) (layer "F.SilkS"))
  (pad "1" thru_hole circle (at 0 0 90) (size 1.5 1.5) (drill 1) (layers "*.Cu" "*.Mask") (remove_unused_layers no) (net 25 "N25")))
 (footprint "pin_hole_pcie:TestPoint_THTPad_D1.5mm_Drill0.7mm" (layer "F.Cu") (at 137.34 81.56 90)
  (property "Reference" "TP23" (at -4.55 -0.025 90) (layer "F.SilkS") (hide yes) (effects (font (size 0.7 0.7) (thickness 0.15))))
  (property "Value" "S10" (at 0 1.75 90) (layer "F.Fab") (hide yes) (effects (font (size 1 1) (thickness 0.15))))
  (fp_circle (center 0 0) (end 0 0.81) (stroke (width 0.12) (type solid)) (fill no) (layer "F.SilkS"))
  (pad "1" thru_hole circle (at 0 0 90) (size 1.5 1.5) (drill 1) (layers "*.Cu" "*.Mask") (remove_unused_layers no) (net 21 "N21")))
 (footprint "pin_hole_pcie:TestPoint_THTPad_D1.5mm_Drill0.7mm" (layer "F.Cu") (at 151.34 81.56 90)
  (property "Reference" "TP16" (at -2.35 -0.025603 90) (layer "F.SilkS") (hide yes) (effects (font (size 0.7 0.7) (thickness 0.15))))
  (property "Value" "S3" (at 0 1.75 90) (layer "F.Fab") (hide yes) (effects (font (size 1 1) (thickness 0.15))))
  (fp_circle (center 0 0) (end 0 0.81) (stroke (width 0.12) (type solid)) (fill no) (layer "F.SilkS"))
  (pad "1" thru_hole circle (at 0 0 90) (size 1.5 1.5) (drill 1) (layers "*.Cu" "*.Mask") (remove_unused_layers no) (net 15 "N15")))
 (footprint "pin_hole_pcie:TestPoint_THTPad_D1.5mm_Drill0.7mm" (layer "F.Cu") (at 169.34 87.56 90)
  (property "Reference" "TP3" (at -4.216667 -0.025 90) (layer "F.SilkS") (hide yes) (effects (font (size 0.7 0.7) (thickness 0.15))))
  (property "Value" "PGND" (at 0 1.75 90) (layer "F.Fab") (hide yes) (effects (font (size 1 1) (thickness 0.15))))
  (fp_circle (center 0 0) (end 0 0.81) (stroke (width 0.12) (type solid)) (fill no) (layer "F.SilkS"))
  (pad "1" thru_hole circle (at 0 0 90) (size 1.5 1.5) (drill 1) (layers "*.Cu" "*.Mask") (remove_unused_layers no) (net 4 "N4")))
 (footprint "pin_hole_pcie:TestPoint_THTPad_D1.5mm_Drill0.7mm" (layer "F.Cu") (at 149.34 81.56 90)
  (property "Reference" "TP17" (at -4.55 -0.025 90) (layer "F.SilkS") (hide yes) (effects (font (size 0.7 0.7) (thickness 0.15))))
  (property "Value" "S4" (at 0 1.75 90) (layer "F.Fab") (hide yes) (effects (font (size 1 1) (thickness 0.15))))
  (fp_circle (center 0 0) (end 0 0.81) (stroke (width 0.12) (type solid)) (fill no) (layer "F.SilkS"))
  (pad "1" thru_hole circle (at 0 0 90) (size 1.5 1.5) (drill 1) (layers "*.Cu" "*.Mask") (remove_unused_layers no) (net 16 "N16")))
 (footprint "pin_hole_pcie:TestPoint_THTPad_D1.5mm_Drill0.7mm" (layer "F.Cu") (at 121.34 81.56 90)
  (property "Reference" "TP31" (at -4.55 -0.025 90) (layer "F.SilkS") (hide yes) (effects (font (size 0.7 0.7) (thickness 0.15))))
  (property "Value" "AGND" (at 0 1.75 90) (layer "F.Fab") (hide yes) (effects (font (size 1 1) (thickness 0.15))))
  (fp_circle (center 0 0) (end 0 0.81) (stroke (width 0.12) (type solid)) (fill no) (layer "F.SilkS"))
  (pad "1" thru_hole circle (at 0 0 90) (size 1.5 1.5) (drill 1) (layers "*.Cu" "*.Mask") (remove_unused_layers no) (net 26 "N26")))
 (gr_line (start 117.9 91.3) (end 123.4 91.3) (stroke (width 0.1) (type solid)) (layer "F.SilkS"))
 (gr_line (start 162.4 91.8) (end 167.9 91.8) (stroke (width 0.2) (type solid)) (layer "F.SilkS"))
 (gr_line (start 148.4 98) (end 148.4 95) (stroke (width 0.1) (type solid)) (layer "F.SilkS"))
 (gr_arc (start 167.9 96) (mid 167.314214 97.414214) (end 165.9 98) (stroke (width 0.05) (type default)) (layer "Edge.Cuts"))
 (gr_line (start 165.9 98) (end 119.9 98) (stroke (width 0.05) (type default)) (layer "Edge.Cuts"))
 (gr_line (start 167.9 80) (end 167.9 96) (stroke (width 0.05) (type solid)) (layer "Edge.Cuts"))
 (gr_line (start 117.9 80) (end 167.9 80) (stroke (width 0.05) (type default)) (layer "Edge.Cuts"))
 (gr_arc (start 119.9 98) (mid 118.485786 97.414214) (end 117.9 96) (stroke (width 0.05) (type default)) (layer "Edge.Cuts"))
 (gr_line (start 117.9 96) (end 117.9 80) (stroke (width 0.05) (type default)) (layer "Edge.Cuts"))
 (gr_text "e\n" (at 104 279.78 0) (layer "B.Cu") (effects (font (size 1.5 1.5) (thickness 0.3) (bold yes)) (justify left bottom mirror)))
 (segment (start 159.4 92.55) (end 159.4 90.05) (width 0.4) (layer "F.Cu") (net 1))
 (segment (start 157.4 90.05) (end 157.4 92.55) (width 0.4) (layer "F.Cu") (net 4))
 (segment (start 157.4 93.55) (end 156.4 94.55) (width 0.4) (layer "F.Cu") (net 4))
 (segment (start 155.4 92.55) (end 155.4 90.05) (width 0.4) (layer "F.Cu") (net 4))
 (segment (start 158.4 88.05) (end 156.4 88.05) (width 0.4) (layer "F.Cu") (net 4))
 (segment (start 155.4 93.55) (end 156.4 94.55) (width 0.4) (layer "F.Cu") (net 4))
 (segment (start 157.4 89.05) (end 156.4 88.05) (width 0.4) (layer "F.Cu") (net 4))
 (segment (start 158.4 94.55) (end 158.4 93.55) (width 0.4) (layer "F.Cu") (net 4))
 (segment (start 158.4 89.05) (end 157.4 90.05) (width 0.4) (layer "F.Cu") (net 4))
 (segment (start 157.4 90.05) (end 157.4 89.05) (width 0.4) (layer "F.Cu") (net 4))
 (segment (start 158.4 94.55) (end 156.4 94.55) (width 0.4) (layer "F.Cu") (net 4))
 (segment (start 158.4 88.05) (end 158.4 89.05) (width 0.4) (layer "F.Cu") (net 4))
 (segment (start 158.4 93.55) (end 157.4 92.55) (width 0.4) (layer "F.Cu") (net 4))
 (segment (start 155.4 90.05) (end 155.4 89.05) (width 0.4) (layer "F.Cu") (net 4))
 (segment (start 157.4 92.55) (end 157.4 93.55) (width 0.4) (layer "F.Cu") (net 4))
 (segment (start 155.4 89.05) (end 156.4 88.05) (width 0.4) (layer "F.Cu") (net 4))
 (segment (start 155.4 92.55) (end 155.4 93.55) (width 0.4) (layer "F.Cu") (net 4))
 (segment (start 154.4 88.05) (end 154.4 94.55) (width 0.4) (layer "F.Cu") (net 10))
 (segment (start 153.4 92.55) (end 153.4 90.05) (width 0.4) (layer "F.Cu") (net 11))
 (segment (start 152.4 94.55) (end 152.4 88.05) (width 0.4) (layer "F.Cu") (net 11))
 (segment (start 151.4 92.55) (end 151.4 90.05) (width 0.4) (layer "F.Cu") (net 11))
 (segment (start 150.4 94.55) (end 150.4 88.05) (width 0.4) (layer "F.Cu") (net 12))
 (segment (start 149.4 92.55) (end 149.4 90.05) (width 0.4) (layer "F.Cu") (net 7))
 (segment (start 146.4 94.55) (end 146.4 88.05) (width 0.3) (layer "F.Cu") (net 3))
 (segment (start 145.4 90.05) (end 145.4 92.55) (width 0.4) (layer "F.Cu") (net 5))
 (segment (start 144.4 88.05) (end 144.4 94.55) (width 0.4) (layer "F.Cu") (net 13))
 (segment (start 143.4 92.55) (end 143.4 90.05) (width 0.4) (layer "F.Cu") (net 14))
 (segment (start 142.4 88.05) (end 142.4 94.55) (width 0.4) (layer "F.Cu") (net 15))
 (segment (start 141.4 92.55) (end 141.4 90.05) (width 0.4) (layer "F.Cu") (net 16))
 (segment (start 140.4 94.55) (end 140.4 88.05) (width 0.4) (layer "F.Cu") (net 17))
 (segment (start 139.4 92.55) (end 139.4 90.05) (width 0.4) (layer "F.Cu") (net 2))
 (segment (start 138.4 94.55) (end 138.4 88.05) (width 0.4) (layer "F.Cu") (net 18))
 (segment (start 137.4 92.55) (end 137.4 90.05) (width 0.4) (layer "F.Cu") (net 19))
 (segment (start 136.4 94.55) (end 136.4 88.05) (width 0.4) (layer "F.Cu") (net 20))
 (segment (start 135.4 92.55) (end 135.4 90.05) (width 0.4) (layer "F.Cu") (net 21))
 (segment (start 134.4 94.55) (end 134.4 88.05) (width 0.4) (layer "F.Cu") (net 6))
 (segment (start 133.4 92.55) (end 133.4 90.05) (width 0.4) (layer "F.Cu") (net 22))
 (segment (start 132.4 94.55) (end 132.4 88.05) (width 0.4) (layer "F.Cu") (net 8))
 (segment (start 131.4 92.55) (end 131.4 90.05) (width 0.4) (layer "F.Cu") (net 9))
 (segment (start 130.4 94.55) (end 130.4 88.05) (width 0.4) (layer "F.Cu") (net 23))
 (segment (start 129.4 92.55) (end 129.4 90.05) (width 0.4) (layer "F.Cu") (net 24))
 (segment (start 128.4 94.55) (end 128.4 88.05) (width 0.4) (layer "F.Cu") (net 25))
 (segment (start 127.4 92.55) (end 127.4 90.05) (width 0.4) (layer "F.Cu") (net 26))
 (segment (start 126.4 94.55) (end 126.4 88.05) (width 0.4) (layer "F.Cu") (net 27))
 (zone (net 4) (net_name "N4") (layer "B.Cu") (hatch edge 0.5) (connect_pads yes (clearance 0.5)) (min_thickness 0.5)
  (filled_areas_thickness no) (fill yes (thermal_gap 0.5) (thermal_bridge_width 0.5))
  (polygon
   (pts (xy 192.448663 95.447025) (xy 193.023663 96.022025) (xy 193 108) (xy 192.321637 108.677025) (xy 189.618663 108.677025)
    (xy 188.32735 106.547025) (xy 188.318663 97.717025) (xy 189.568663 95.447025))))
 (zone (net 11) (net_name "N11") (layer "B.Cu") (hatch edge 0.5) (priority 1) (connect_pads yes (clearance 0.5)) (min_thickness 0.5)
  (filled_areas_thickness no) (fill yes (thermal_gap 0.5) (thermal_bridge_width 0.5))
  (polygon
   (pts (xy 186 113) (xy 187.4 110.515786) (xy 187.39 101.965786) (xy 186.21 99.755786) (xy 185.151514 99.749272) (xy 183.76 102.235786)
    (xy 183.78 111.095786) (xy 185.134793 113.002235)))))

